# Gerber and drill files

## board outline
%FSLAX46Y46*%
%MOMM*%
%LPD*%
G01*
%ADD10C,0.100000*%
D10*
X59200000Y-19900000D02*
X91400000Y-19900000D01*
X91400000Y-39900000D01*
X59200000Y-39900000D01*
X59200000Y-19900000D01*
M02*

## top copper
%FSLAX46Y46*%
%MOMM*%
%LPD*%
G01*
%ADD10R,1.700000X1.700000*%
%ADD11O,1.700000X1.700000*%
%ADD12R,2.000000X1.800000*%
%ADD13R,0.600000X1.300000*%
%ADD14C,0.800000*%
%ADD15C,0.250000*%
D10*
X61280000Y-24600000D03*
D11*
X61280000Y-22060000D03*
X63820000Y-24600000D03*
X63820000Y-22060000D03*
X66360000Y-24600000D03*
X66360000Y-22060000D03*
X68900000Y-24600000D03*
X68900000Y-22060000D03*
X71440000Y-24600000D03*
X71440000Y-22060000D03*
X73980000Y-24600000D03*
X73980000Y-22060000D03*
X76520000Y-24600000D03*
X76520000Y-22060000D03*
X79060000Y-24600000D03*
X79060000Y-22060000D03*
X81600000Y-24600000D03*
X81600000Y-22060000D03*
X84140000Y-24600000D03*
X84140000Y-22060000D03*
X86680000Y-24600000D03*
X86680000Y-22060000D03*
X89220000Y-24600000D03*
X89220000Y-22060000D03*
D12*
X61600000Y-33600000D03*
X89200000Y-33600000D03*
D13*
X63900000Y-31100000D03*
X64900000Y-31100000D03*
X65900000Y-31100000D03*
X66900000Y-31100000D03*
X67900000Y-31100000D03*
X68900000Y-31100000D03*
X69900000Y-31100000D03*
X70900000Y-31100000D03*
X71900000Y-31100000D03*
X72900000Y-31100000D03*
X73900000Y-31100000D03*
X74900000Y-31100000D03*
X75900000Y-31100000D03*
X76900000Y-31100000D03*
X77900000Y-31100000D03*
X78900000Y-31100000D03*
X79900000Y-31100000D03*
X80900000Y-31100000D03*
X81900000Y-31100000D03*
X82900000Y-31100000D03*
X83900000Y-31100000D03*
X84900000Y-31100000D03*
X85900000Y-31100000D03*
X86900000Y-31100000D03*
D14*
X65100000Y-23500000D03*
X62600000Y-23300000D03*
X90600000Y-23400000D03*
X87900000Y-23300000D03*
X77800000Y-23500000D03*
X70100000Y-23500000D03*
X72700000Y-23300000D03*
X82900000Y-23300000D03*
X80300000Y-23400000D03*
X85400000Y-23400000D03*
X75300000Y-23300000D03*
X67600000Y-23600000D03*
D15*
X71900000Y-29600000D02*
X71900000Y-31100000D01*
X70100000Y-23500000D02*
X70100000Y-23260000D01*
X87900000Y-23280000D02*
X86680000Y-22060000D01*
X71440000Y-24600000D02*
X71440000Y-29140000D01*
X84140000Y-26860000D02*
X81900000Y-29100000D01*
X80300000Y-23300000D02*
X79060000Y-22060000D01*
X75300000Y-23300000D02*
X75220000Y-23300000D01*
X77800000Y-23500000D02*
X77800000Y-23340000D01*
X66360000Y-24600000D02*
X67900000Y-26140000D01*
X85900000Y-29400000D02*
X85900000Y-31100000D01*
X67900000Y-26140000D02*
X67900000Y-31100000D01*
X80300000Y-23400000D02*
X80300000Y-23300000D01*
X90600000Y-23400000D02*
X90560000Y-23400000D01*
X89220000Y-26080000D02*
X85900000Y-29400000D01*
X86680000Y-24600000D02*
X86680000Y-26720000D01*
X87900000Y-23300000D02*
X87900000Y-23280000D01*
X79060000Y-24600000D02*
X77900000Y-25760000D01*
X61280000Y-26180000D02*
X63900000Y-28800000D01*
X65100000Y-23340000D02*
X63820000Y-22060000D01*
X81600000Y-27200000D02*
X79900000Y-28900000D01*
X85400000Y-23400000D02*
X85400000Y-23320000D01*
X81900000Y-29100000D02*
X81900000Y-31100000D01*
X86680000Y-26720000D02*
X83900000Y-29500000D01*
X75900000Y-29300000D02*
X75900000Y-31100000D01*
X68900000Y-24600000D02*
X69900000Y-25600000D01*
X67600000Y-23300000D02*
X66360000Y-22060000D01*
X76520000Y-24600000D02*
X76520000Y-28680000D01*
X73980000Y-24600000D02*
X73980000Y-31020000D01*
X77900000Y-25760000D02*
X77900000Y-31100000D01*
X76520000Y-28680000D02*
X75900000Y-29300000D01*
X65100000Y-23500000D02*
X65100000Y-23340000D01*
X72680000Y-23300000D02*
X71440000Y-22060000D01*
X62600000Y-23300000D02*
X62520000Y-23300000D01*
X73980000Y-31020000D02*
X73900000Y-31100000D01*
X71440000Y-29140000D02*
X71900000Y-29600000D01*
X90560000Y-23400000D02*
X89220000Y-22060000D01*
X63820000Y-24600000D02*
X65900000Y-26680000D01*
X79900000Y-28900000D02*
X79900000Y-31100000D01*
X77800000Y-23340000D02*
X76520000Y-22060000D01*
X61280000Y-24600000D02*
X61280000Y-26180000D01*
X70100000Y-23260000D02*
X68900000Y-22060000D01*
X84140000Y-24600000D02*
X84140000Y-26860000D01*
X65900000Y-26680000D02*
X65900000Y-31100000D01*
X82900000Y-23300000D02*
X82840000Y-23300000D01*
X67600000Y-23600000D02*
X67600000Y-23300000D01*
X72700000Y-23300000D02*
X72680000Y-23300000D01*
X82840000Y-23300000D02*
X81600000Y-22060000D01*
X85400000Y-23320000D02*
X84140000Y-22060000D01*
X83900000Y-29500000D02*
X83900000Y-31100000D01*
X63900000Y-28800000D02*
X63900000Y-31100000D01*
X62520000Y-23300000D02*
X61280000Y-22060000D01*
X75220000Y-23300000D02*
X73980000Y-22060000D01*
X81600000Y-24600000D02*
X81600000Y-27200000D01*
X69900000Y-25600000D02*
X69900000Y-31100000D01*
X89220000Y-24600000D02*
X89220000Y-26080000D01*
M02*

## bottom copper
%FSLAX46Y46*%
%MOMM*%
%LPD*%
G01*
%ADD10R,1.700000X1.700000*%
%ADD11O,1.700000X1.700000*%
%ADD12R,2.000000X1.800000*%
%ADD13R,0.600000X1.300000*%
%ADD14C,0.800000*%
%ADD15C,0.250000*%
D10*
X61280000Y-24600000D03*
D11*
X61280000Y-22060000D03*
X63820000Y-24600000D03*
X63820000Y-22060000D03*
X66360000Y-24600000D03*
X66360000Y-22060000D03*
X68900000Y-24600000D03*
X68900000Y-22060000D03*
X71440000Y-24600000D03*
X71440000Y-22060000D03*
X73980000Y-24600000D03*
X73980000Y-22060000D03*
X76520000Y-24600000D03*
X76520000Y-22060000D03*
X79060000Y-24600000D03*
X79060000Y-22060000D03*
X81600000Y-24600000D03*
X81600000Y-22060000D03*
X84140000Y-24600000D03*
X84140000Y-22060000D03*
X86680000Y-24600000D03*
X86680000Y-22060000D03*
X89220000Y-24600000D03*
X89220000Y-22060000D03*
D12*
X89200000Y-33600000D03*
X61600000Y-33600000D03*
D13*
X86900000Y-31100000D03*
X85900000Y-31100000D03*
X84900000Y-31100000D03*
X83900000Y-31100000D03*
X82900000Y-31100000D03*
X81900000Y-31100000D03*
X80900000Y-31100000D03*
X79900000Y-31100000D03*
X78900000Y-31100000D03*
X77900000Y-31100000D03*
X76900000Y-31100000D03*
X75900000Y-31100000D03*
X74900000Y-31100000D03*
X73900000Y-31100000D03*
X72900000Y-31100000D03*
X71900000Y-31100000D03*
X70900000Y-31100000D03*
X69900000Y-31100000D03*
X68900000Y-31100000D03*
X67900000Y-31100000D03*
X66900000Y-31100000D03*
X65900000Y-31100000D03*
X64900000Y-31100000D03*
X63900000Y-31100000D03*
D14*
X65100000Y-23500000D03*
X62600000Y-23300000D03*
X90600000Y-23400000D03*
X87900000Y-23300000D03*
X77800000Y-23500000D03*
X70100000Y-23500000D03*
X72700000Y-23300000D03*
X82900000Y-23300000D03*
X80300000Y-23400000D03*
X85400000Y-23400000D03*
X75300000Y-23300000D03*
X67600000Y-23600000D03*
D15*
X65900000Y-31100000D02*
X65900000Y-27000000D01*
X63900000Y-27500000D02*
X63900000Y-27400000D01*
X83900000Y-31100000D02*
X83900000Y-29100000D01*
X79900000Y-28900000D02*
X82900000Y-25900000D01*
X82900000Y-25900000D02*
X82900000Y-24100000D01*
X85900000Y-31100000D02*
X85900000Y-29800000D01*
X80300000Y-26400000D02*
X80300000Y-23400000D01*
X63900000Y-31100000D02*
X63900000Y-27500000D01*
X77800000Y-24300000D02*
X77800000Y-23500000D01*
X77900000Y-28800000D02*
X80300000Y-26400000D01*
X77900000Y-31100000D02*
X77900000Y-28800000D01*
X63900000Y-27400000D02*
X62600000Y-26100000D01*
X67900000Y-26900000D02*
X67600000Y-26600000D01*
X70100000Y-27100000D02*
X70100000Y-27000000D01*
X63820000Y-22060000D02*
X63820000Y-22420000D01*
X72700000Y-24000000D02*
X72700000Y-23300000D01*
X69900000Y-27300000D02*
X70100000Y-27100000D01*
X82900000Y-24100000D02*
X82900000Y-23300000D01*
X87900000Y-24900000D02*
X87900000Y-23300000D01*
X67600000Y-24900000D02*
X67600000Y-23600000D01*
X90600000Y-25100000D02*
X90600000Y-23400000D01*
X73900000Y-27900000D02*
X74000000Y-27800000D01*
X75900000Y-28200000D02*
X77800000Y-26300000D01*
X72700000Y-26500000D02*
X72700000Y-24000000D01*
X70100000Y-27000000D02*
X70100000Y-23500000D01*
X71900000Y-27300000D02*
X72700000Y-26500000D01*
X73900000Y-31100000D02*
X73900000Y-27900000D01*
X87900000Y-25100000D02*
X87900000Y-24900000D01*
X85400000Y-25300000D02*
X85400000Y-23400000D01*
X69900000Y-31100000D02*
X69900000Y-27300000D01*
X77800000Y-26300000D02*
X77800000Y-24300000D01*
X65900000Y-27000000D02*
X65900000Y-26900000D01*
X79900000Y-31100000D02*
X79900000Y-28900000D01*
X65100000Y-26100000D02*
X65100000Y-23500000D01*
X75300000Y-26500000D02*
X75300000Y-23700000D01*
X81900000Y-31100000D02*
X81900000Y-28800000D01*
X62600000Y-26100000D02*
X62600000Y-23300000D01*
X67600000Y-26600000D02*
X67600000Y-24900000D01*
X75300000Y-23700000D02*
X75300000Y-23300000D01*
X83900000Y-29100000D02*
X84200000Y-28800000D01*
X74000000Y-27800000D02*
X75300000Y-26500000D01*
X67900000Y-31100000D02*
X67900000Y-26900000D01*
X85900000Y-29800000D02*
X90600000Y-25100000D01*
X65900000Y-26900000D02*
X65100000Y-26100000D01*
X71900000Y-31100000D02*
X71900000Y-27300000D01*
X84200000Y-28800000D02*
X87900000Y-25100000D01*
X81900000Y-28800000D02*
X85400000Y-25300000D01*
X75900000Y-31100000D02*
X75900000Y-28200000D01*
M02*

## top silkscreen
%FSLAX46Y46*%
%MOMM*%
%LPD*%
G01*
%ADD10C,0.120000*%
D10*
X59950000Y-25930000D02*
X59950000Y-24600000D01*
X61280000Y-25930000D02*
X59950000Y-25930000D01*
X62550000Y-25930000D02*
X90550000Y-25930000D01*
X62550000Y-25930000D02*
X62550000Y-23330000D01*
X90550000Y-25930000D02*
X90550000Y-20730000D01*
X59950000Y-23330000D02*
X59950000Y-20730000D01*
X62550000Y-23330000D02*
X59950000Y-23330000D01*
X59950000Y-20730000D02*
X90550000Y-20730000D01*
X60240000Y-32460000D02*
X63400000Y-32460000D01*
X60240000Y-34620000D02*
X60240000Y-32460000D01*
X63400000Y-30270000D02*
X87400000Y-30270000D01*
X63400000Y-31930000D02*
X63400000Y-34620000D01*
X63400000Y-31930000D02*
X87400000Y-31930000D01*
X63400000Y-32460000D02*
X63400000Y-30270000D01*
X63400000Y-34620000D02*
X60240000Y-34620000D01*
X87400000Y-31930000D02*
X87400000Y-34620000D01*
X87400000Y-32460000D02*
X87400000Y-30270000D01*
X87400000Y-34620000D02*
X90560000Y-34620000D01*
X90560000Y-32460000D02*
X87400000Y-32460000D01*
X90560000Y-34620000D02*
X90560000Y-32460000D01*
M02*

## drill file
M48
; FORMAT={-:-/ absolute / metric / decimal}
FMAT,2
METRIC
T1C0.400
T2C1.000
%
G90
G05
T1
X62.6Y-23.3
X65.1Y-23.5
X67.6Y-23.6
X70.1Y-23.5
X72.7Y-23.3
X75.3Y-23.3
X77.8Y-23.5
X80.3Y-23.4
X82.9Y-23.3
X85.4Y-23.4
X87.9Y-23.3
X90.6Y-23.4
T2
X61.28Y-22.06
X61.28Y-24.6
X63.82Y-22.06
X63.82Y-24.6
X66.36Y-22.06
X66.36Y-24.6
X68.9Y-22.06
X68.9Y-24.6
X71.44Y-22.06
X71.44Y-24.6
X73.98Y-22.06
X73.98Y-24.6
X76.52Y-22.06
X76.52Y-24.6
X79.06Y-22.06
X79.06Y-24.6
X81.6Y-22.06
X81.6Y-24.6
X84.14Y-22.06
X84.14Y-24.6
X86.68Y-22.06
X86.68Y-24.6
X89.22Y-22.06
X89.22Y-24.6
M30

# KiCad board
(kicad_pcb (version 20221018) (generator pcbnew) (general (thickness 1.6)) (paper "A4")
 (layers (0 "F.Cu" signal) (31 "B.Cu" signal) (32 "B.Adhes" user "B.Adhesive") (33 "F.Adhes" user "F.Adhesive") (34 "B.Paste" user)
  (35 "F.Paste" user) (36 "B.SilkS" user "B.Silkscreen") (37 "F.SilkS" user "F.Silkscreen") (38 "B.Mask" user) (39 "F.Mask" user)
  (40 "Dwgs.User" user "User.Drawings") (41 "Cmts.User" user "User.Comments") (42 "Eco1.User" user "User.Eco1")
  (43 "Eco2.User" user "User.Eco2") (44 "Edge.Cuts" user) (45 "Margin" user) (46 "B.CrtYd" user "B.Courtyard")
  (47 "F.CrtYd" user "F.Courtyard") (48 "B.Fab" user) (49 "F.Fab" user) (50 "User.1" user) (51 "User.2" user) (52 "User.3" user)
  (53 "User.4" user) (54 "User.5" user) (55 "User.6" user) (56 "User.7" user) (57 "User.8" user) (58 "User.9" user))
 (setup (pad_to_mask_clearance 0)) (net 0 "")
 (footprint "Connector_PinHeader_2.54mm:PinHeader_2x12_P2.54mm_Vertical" (layer "F.Cu") (at 61.28 24.6 90)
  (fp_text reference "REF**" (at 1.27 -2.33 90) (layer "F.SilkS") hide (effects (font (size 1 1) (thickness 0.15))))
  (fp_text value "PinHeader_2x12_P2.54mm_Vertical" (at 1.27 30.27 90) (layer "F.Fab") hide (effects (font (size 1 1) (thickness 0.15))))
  (fp_line (start -1.33 -1.33) (end 0 -1.33) (stroke (width 0.12) (type solid)) (layer "F.SilkS"))
  (fp_line (start -1.33 0) (end -1.33 -1.33) (stroke (width 0.12) (type solid)) (layer "F.SilkS"))
  (fp_line (start -1.33 1.27) (end -1.33 29.27) (stroke (width 0.12) (type solid)) (layer "F.SilkS"))
  (fp_line (start -1.33 1.27) (end 1.27 1.27) (stroke (width 0.12) (type solid)) (layer "F.SilkS"))
  (fp_line (start -1.33 29.27) (end 3.87 29.27) (stroke (width 0.12) (type solid)) (layer "F.SilkS"))
  (fp_line (start 1.27 -1.33) (end 3.87 -1.33) (stroke (width 0.12) (type solid)) (layer "F.SilkS"))
  (fp_line (start 1.27 1.27) (end 1.27 -1.33) (stroke (width 0.12) (type solid)) (layer "F.SilkS"))
  (fp_line (start 3.87 -1.33) (end 3.87 29.27) (stroke (width 0.12) (type solid)) (layer "F.SilkS"))
  (pad "1" thru_hole rect (at 0 0 90) (size 1.7 1.7) (drill 1) (layers "*.Cu" "*.Mask"))
  (pad "2" thru_hole oval (at 2.54 0 90) (size 1.7 1.7) (drill 1) (layers "*.Cu" "*.Mask"))
  (pad "3" thru_hole oval (at 0 2.54 90) (size 1.7 1.7) (drill 1) (layers "*.Cu" "*.Mask"))
  (pad "4" thru_hole oval (at 2.54 2.54 90) (size 1.7 1.7) (drill 1) (layers "*.Cu" "*.Mask"))
  (pad "5" thru_hole oval (at 0 5.08 90) (size 1.7 1.7) (drill 1) (layers "*.Cu" "*.Mask"))
  (pad "6" thru_hole oval (at 2.54 5.08 90) (size 1.7 1.7) (drill 1) (layers "*.Cu" "*.Mask"))
  (pad "7" thru_hole oval (at 0 7.62 90) (size 1.7 1.7) (drill 1) (layers "*.Cu" "*.Mask"))
  (pad "8" thru_hole oval (at 2.54 7.62 90) (size 1.7 1.7) (drill 1) (layers "*.Cu" "*.Mask"))
  (pad "9" thru_hole oval (at 0 10.16 90) (size 1.7 1.7) (drill 1) (layers "*.Cu" "*.Mask"))
  (pad "10" thru_hole oval (at 2.54 10.16 90) (size 1.7 1.7) (drill 1) (layers "*.Cu" "*.Mask"))
  (pad "11" thru_hole oval (at 0 12.7 90) (size 1.7 1.7) (drill 1) (layers "*.Cu" "*.Mask"))
  (pad "12" thru_hole oval (at 2.54 12.7 90) (size 1.7 1.7) (drill 1) (layers "*.Cu" "*.Mask"))
  (pad "13" thru_hole oval (at 0 15.24 90) (size 1.7 1.7) (drill 1) (layers "*.Cu" "*.Mask"))
  (pad "14" thru_hole oval (at 2.54 15.24 90) (size 1.7 1.7) (drill 1) (layers "*.Cu" "*.Mask"))
  (pad "15" thru_hole oval (at 0 17.78 90) (size 1.7 1.7) (drill 1) (layers "*.Cu" "*.Mask"))
  (pad "16" thru_hole oval (at 2.54 17.78 90) (size 1.7 1.7) (drill 1) (layers "*.Cu" "*.Mask"))
  (pad "17" thru_hole oval (at 0 20.32 90) (size 1.7 1.7) (drill 1) (layers "*.Cu" "*.Mask"))
  (pad "18" thru_hole oval (at 2.54 20.32 90) (size 1.7 1.7) (drill 1) (layers "*.Cu" "*.Mask"))
  (pad "19" thru_hole oval (at 0 22.86 90) (size 1.7 1.7) (drill 1) (layers "*.Cu" "*.Mask"))
  (pad "20" thru_hole oval (at 2.54 22.86 90) (size 1.7 1.7) (drill 1) (layers "*.Cu" "*.Mask"))
  (pad "21" thru_hole oval (at 0 25.4 90) (size 1.7 1.7) (drill 1) (layers "*.Cu" "*.Mask"))
  (pad "22" thru_hole oval (at 2.54 25.4 90) (size 1.7 1.7) (drill 1) (layers "*.Cu" "*.Mask"))
  (pad "23" thru_hole oval (at 0 27.94 90) (size 1.7 1.7) (drill 1) (layers "*.Cu" "*.Mask"))
  (pad "24" thru_hole oval (at 2.54 27.94 90) (size 1.7 1.7) (drill 1) (layers "*.Cu" "*.Mask")))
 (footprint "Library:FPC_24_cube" (layer "F.Cu") (at 75.4 31.1)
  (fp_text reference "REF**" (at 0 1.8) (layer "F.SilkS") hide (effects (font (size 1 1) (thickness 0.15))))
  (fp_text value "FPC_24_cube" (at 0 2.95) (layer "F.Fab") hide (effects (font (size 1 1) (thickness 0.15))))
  (fp_line (start -15.16 1.36) (end -12 1.36) (stroke (width 0.12) (type default)) (layer "F.SilkS"))
  (fp_line (start -15.16 3.52) (end -15.16 1.36) (stroke (width 0.12) (type default)) (layer "F.SilkS"))
  (fp_line (start -12 -0.83) (end 12 -0.83) (stroke (width 0.12) (type default)) (layer "F.SilkS"))
  (fp_line (start -12 0.83) (end -12 3.52) (stroke (width 0.12) (type default)) (layer "F.SilkS"))
  (fp_line (start -12 0.83) (end 12 0.83) (stroke (width 0.12) (type default)) (layer "F.SilkS"))
  (fp_line (start -12 1.36) (end -12 -0.83) (stroke (width 0.12) (type default)) (layer "F.SilkS"))
  (fp_line (start -12 3.52) (end -15.16 3.52) (stroke (width 0.12) (type default)) (layer "F.SilkS"))
  (fp_line (start 12 0.83) (end 12 3.52) (stroke (width 0.12) (type default)) (layer "F.SilkS"))
  (fp_line (start 12 1.36) (end 12 -0.83) (stroke (width 0.12) (type default)) (layer "F.SilkS"))
  (fp_line (start 12 3.52) (end 15.16 3.52) (stroke (width 0.12) (type default)) (layer "F.SilkS"))
  (fp_line (start 15.16 1.36) (end 12 1.36) (stroke (width 0.12) (type default)) (layer "F.SilkS"))
  (fp_line (start 15.16 3.52) (end 15.16 1.36) (stroke (width 0.12) (type default)) (layer "F.SilkS"))
  (pad "0" smd rect (at -13.8 2.5) (size 2 1.8) (layers "F.Cu" "F.Paste" "F.Mask") (thermal_bridge_angle 45))
  (pad "0" smd rect (at 13.8 2.5) (size 2 1.8) (layers "F.Cu" "F.Paste" "F.Mask") (thermal_bridge_angle 45))
  (pad "1" smd rect (at -11.5 0) (size 0.6 1.3) (layers "F.Cu" "F.Paste" "F.Mask") (thermal_bridge_angle 45))
  (pad "2" smd rect (at -10.5 0) (size 0.6 1.3) (layers "F.Cu" "F.Paste" "F.Mask") (thermal_bridge_angle 45))
  (pad "3" smd rect (at -9.5 0) (size 0.6 1.3) (layers "F.Cu" "F.Paste" "F.Mask") (thermal_bridge_angle 45))
  (pad "4" smd rect (at -8.5 0) (size 0.6 1.3) (layers "F.Cu" "F.Paste" "F.Mask") (thermal_bridge_angle 45))
  (pad "5" smd rect (at -7.5 0) (size 0.6 1.3) (layers "F.Cu" "F.Paste" "F.Mask") (thermal_bridge_angle 45))
  (pad "6" smd rect (at -6.5 0) (size 0.6 1.3) (layers "F.Cu" "F.Paste" "F.Mask") (thermal_bridge_angle 45))
  (pad "7" smd rect (at -5.5 0) (size 0.6 1.3) (layers "F.Cu" "F.Paste" "F.Mask") (thermal_bridge_angle 45))
  (pad "8" smd rect (at -4.5 0) (size 0.6 1.3) (layers "F.Cu" "F.Paste" "F.Mask") (thermal_bridge_angle 45))
  (pad "9" smd rect (at -3.5 0) (size 0.6 1.3) (layers "F.Cu" "F.Paste" "F.Mask") (thermal_bridge_angle 45))
  (pad "10" smd rect (at -2.5 0) (size 0.6 1.3) (layers "F.Cu" "F.Paste" "F.Mask") (thermal_bridge_angle 45))
  (pad "11" smd rect (at -1.5 0) (size 0.6 1.3) (layers "F.Cu" "F.Paste" "F.Mask") (thermal_bridge_angle 45))
  (pad "12" smd rect (at -0.5 0) (size 0.6 1.3) (layers "F.Cu" "F.Paste" "F.Mask") (thermal_bridge_angle 45))
  (pad "13" smd rect (at 0.5 0) (size 0.6 1.3) (layers "F.Cu" "F.Paste" "F.Mask") (thermal_bridge_angle 45))
  (pad "14" smd rect (at 1.5 0) (size 0.6 1.3) (layers "F.Cu" "F.Paste" "F.Mask") (thermal_bridge_angle 45))
  (pad "15" smd rect (at 2.5 0) (size 0.6 1.3) (layers "F.Cu" "F.Paste" "F.Mask") (thermal_bridge_angle 45))
  (pad "16" smd rect (at 3.5 0) (size 0.6 1.3) (layers "F.Cu" "F.Paste" "F.Mask") (thermal_bridge_angle 45))
  (pad "17" smd rect (at 4.5 0) (size 0.6 1.3) (layers "F.Cu" "F.Paste" "F.Mask") (thermal_bridge_angle 45))
  (pad "18" smd rect (at 5.5 0) (size 0.6 1.3) (layers "F.Cu" "F.Paste" "F.Mask") (thermal_bridge_angle 45))
  (pad "19" smd rect (at 6.5 0) (size 0.6 1.3) (layers "F.Cu" "F.Paste" "F.Mask") (thermal_bridge_angle 45))
  (pad "20" smd rect (at 7.5 0) (size 0.6 1.3) (layers "F.Cu" "F.Paste" "F.Mask") (thermal_bridge_angle 45))
  (pad "21" smd rect (at 8.5 0) (size 0.6 1.3) (layers "F.Cu" "F.Paste" "F.Mask") (thermal_bridge_angle 45))
  (pad "22" smd rect (at 9.5 0) (size 0.6 1.3) (layers "F.Cu" "F.Paste" "F.Mask") (thermal_bridge_angle 45))
  (pad "23" smd rect (at 10.5 0) (size 0.6 1.3) (layers "F.Cu" "F.Paste" "F.Mask") (thermal_bridge_angle 45))
  (pad "24" smd rect (at 11.5 0) (size 0.6 1.3) (layers "F.Cu" "F.Paste" "F.Mask") (thermal_bridge_angle 45)))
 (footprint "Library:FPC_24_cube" (layer "B.Cu") (at 75.4 31.1 180)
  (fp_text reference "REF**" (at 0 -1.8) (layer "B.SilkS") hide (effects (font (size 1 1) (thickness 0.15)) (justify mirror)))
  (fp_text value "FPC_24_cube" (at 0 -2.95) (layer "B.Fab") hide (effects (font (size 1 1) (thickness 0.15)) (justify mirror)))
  (pad "0" smd rect (at -13.8 -2.5 180) (size 2 1.8) (layers "B.Cu" "B.Paste" "B.Mask") (thermal_bridge_angle 45))
  (pad "0" smd rect (at 13.8 -2.5 180) (size 2 1.8) (layers "B.Cu" "B.Paste" "B.Mask") (thermal_bridge_angle 45))
  (pad "1" smd rect (at -11.5 0 180) (size 0.6 1.3) (layers "B.Cu" "B.Paste" "B.Mask") (thermal_bridge_angle 45))
  (pad "2" smd rect (at -10.5 0 180) (size 0.6 1.3) (layers "B.Cu" "B.Paste" "B.Mask") (thermal_bridge_angle 45))
  (pad "3" smd rect (at -9.5 0 180) (size 0.6 1.3) (layers "B.Cu" "B.Paste" "B.Mask") (thermal_bridge_angle 45))
  (pad "4" smd rect (at -8.5 0 180) (size 0.6 1.3) (layers "B.Cu" "B.Paste" "B.Mask") (thermal_bridge_angle 45))
  (pad "5" smd rect (at -7.5 0 180) (size 0.6 1.3) (layers "B.Cu" "B.Paste" "B.Mask") (thermal_bridge_angle 45))
  (pad "6" smd rect (at -6.5 0 180) (size 0.6 1.3) (layers "B.Cu" "B.Paste" "B.Mask") (thermal_bridge_angle 45))
  (pad "7" smd rect (at -5.5 0 180) (size 0.6 1.3) (layers "B.Cu" "B.Paste" "B.Mask") (thermal_bridge_angle 45))
  (pad "8" smd rect (at -4.5 0 180) (size 0.6 1.3) (layers "B.Cu" "B.Paste" "B.Mask") (thermal_bridge_angle 45))
  (pad "9" smd rect (at -3.5 0 180) (size 0.6 1.3) (layers "B.Cu" "B.Paste" "B.Mask") (thermal_bridge_angle 45))
  (pad "10" smd rect (at -2.5 0 180) (size 0.6 1.3) (layers "B.Cu" "B.Paste" "B.Mask") (thermal_bridge_angle 45))
  (pad "11" smd rect (at -1.5 0 180) (size 0.6 1.3) (layers "B.Cu" "B.Paste" "B.Mask") (thermal_bridge_angle 45))
  (pad "12" smd rect (at -0.5 0 180) (size 0.6 1.3) (layers "B.Cu" "B.Paste" "B.Mask") (thermal_bridge_angle 45))
  (pad "13" smd rect (at 0.5 0 180) (size 0.6 1.3) (layers "B.Cu" "B.Paste" "B.Mask") (thermal_bridge_angle 45))
  (pad "14" smd rect (at 1.5 0 180) (size 0.6 1.3) (layers "B.Cu" "B.Paste" "B.Mask") (thermal_bridge_angle 45))
  (pad "15" smd rect (at 2.5 0 180) (size 0.6 1.3) (layers "B.Cu" "B.Paste" "B.Mask") (thermal_bridge_angle 45))
  (pad "16" smd rect (at 3.5 0 180) (size 0.6 1.3) (layers "B.Cu" "B.Paste" "B.Mask") (thermal_bridge_angle 45))
  (pad "17" smd rect (at 4.5 0 180) (size 0.6 1.3) (layers "B.Cu" "B.Paste" "B.Mask") (thermal_bridge_angle 45))
  (pad "18" smd rect (at 5.5 0 180) (size 0.6 1.3) (layers "B.Cu" "B.Paste" "B.Mask") (thermal_bridge_angle 45))
  (pad "19" smd rect (at 6.5 0 180) (size 0.6 1.3) (layers "B.Cu" "B.Paste" "B.Mask") (thermal_bridge_angle 45))
  (pad "20" smd rect (at 7.5 0 180) (size 0.6 1.3) (layers "B.Cu" "B.Paste" "B.Mask") (thermal_bridge_angle 45))
  (pad "21" smd rect (at 8.5 0 180) (size 0.6 1.3) (layers "B.Cu" "B.Paste" "B.Mask") (thermal_bridge_angle 45))
  (pad "22" smd rect (at 9.5 0 180) (size 0.6 1.3) (layers "B.Cu" "B.Paste" "B.Mask") (thermal_bridge_angle 45))
  (pad "23" smd rect (at 10.5 0 180) (size 0.6 1.3) (layers "B.Cu" "B.Paste" "B.Mask") (thermal_bridge_angle 45))
  (pad "24" smd rect (at 11.5 0 180) (size 0.6 1.3) (layers "B.Cu" "B.Paste" "B.Mask") (thermal_bridge_angle 45)))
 (gr_rect (start 59.2 19.9) (end 91.4 39.9) (stroke (width 0.1) (type default)) (fill none) (layer "Edge.Cuts"))
 (segment (start 71.9 29.6) (end 71.9 31.1) (width 0.25) (layer "F.Cu") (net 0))
 (segment (start 70.1 23.5) (end 70.1 23.26) (width 0.25) (layer "F.Cu") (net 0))
 (segment (start 87.9 23.28) (end 86.68 22.06) (width 0.25) (layer "F.Cu") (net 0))
 (segment (start 71.44 24.6) (end 71.44 29.14) (width 0.25) (layer "F.Cu") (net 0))
 (segment (start 84.14 26.86) (end 81.9 29.1) (width 0.25) (layer "F.Cu") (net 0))
 (segment (start 80.3 23.3) (end 79.06 22.06) (width 0.25) (layer "F.Cu") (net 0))
 (segment (start 75.3 23.3) (end 75.22 23.3) (width 0.25) (layer "F.Cu") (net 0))
 (segment (start 77.8 23.5) (end 77.8 23.34) (width 0.25) (layer "F.Cu") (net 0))
 (segment (start 66.36 24.6) (end 67.9 26.14) (width 0.25) (layer "F.Cu") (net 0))
 (segment (start 85.9 29.4) (end 85.9 31.1) (width 0.25) (layer "F.Cu") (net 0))
 (segment (start 67.9 26.14) (end 67.9 31.1) (width 0.25) (layer "F.Cu") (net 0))
 (segment (start 80.3 23.4) (end 80.3 23.3) (width 0.25) (layer "F.Cu") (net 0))
 (segment (start 90.6 23.4) (end 90.56 23.4) (width 0.25) (layer "F.Cu") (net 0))
 (segment (start 89.22 26.08) (end 85.9 29.4) (width 0.25) (layer "F.Cu") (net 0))
 (segment (start 86.68 24.6) (end 86.68 26.72) (width 0.25) (layer "F.Cu") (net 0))
 (segment (start 87.9 23.3) (end 87.9 23.28) (width 0.25) (layer "F.Cu") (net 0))
 (segment (start 79.06 24.6) (end 77.9 25.76) (width 0.25) (layer "F.Cu") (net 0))
 (segment (start 61.28 26.18) (end 63.9 28.8) (width 0.25) (layer "F.Cu") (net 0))
 (segment (start 65.1 23.34) (end 63.82 22.06) (width 0.25) (layer "F.Cu") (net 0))
 (segment (start 81.6 27.2) (end 79.9 28.9) (width 0.25) (layer "F.Cu") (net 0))
 (segment (start 85.4 23.4) (end 85.4 23.32) (width 0.25) (layer "F.Cu") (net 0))
 (segment (start 81.9 29.1) (end 81.9 31.1) (width 0.25) (layer "F.Cu") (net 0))
 (segment (start 86.68 26.72) (end 83.9 29.5) (width 0.25) (layer "F.Cu") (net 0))
 (segment (start 75.9 29.3) (end 75.9 31.1) (width 0.25) (layer "F.Cu") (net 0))
 (segment (start 68.9 24.6) (end 69.9 25.6) (width 0.25) (layer "F.Cu") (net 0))
 (segment (start 67.6 23.3) (end 66.36 22.06) (width 0.25) (layer "F.Cu") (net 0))
 (segment (start 76.52 24.6) (end 76.52 28.68) (width 0.25) (layer "F.Cu") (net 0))
 (segment (start 73.98 24.6) (end 73.98 31.02) (width 0.25) (layer "F.Cu") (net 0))
 (segment (start 77.9 25.76) (end 77.9 31.1) (width 0.25) (layer "F.Cu") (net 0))
 (segment (start 76.52 28.68) (end 75.9 29.3) (width 0.25) (layer "F.Cu") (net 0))
 (segment (start 65.1 23.5) (end 65.1 23.34) (width 0.25) (layer "F.Cu") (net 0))
 (segment (start 72.68 23.3) (end 71.44 22.06) (width 0.25) (layer "F.Cu") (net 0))
 (segment (start 62.6 23.3) (end 62.52 23.3) (width 0.25) (layer "F.Cu") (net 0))
 (segment (start 73.98 31.02) (end 73.9 31.1) (width 0.25) (layer "F.Cu") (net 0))
 (segment (start 71.44 29.14) (end 71.9 29.6) (width 0.25) (layer "F.Cu") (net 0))
 (segment (start 90.56 23.4) (end 89.22 22.06) (width 0.25) (layer "F.Cu") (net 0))
 (segment (start 63.82 24.6) (end 65.9 26.68) (width 0.25) (layer "F.Cu") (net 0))
 (segment (start 79.9 28.9) (end 79.9 31.1) (width 0.25) (layer "F.Cu") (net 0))
 (segment (start 77.8 23.34) (end 76.52 22.06) (width 0.25) (layer "F.Cu") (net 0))
 (segment (start 61.28 24.6) (end 61.28 26.18) (width 0.25) (layer "F.Cu") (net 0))
 (segment (start 70.1 23.26) (end 68.9 22.06) (width 0.25) (layer "F.Cu") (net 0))
 (segment (start 84.14 24.6) (end 84.14 26.86) (width 0.25) (layer "F.Cu") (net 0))
 (segment (start 65.9 26.68) (end 65.9 31.1) (width 0.25) (layer "F.Cu") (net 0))
 (segment (start 82.9 23.3) (end 82.84 23.3) (width 0.25) (layer "F.Cu") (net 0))
 (segment (start 67.6 23.6) (end 67.6 23.3) (width 0.25) (layer "F.Cu") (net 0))
 (segment (start 72.7 23.3) (end 72.68 23.3) (width 0.25) (layer "F.Cu") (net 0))
 (segment (start 82.84 23.3) (end 81.6 22.06) (width 0.25) (layer "F.Cu") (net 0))
 (segment (start 85.4 23.32) (end 84.14 22.06) (width 0.25) (layer "F.Cu") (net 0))
 (segment (start 83.9 29.5) (end 83.9 31.1) (width 0.25) (layer "F.Cu") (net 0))
 (segment (start 63.9 28.8) (end 63.9 31.1) (width 0.25) (layer "F.Cu") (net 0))
 (segment (start 62.52 23.3) (end 61.28 22.06) (width 0.25) (layer "F.Cu") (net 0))
 (segment (start 75.22 23.3) (end 73.98 22.06) (width 0.25) (layer "F.Cu") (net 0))
 (segment (start 81.6 24.6) (end 81.6 27.2) (width 0.25) (layer "F.Cu") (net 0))
 (segment (start 69.9 25.6) (end 69.9 31.1) (width 0.25) (layer "F.Cu") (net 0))
 (segment (start 89.22 24.6) (end 89.22 26.08) (width 0.25) (layer "F.Cu") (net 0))
 (via (at 65.1 23.5) (size 0.8) (drill 0.4) (layers "F.Cu" "B.Cu") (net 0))
 (via (at 62.6 23.3) (size 0.8) (drill 0.4) (layers "F.Cu" "B.Cu") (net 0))
 (via (at 90.6 23.4) (size 0.8) (drill 0.4) (layers "F.Cu" "B.Cu") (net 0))
 (via (at 87.9 23.3) (size 0.8) (drill 0.4) (layers "F.Cu" "B.Cu") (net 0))
 (via (at 77.8 23.5) (size 0.8) (drill 0.4) (layers "F.Cu" "B.Cu") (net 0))
 (via (at 70.1 23.5) (size 0.8) (drill 0.4) (layers "F.Cu" "B.Cu") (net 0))
 (via (at 72.7 23.3) (size 0.8) (drill 0.4) (layers "F.Cu" "B.Cu") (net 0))
 (via (at 82.9 23.3) (size 0.8) (drill 0.4) (layers "F.Cu" "B.Cu") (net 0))
 (via (at 80.3 23.4) (size 0.8) (drill 0.4) (layers "F.Cu" "B.Cu") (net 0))
 (via (at 85.4 23.4) (size 0.8) (drill 0.4) (layers "F.Cu" "B.Cu") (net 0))
 (via (at 75.3 23.3) (size 0.8) (drill 0.4) (layers "F.Cu" "B.Cu") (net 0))
 (via (at 67.6 23.6) (size 0.8) (drill 0.4) (layers "F.Cu" "B.Cu") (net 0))
 (segment (start 65.9 31.1) (end 65.9 27) (width 0.25) (layer "B.Cu") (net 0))
 (segment (start 63.9 27.5) (end 63.9 27.4) (width 0.25) (layer "B.Cu") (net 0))
 (segment (start 83.9 31.1) (end 83.9 29.1) (width 0.25) (layer "B.Cu") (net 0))
 (segment (start 79.9 28.9) (end 82.9 25.9) (width 0.25) (layer "B.Cu") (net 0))
 (segment (start 82.9 25.9) (end 82.9 24.1) (width 0.25) (layer "B.Cu") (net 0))
 (segment (start 85.9 31.1) (end 85.9 29.8) (width 0.25) (layer "B.Cu") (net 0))
 (segment (start 80.3 26.4) (end 80.3 23.4) (width 0.25) (layer "B.Cu") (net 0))
 (segment (start 63.9 31.1) (end 63.9 27.5) (width 0.25) (layer "B.Cu") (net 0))
 (segment (start 77.8 24.3) (end 77.8 23.5) (width 0.25) (layer "B.Cu") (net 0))
 (segment (start 77.9 28.8) (end 80.3 26.4) (width 0.25) (layer "B.Cu") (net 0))
 (segment (start 77.9 31.1) (end 77.9 28.8) (width 0.25) (layer "B.Cu") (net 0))
 (segment (start 63.9 27.4) (end 62.6 26.1) (width 0.25) (layer "B.Cu") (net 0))
 (segment (start 67.9 26.9) (end 67.6 26.6) (width 0.25) (layer "B.Cu") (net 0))
 (segment (start 70.1 27.1) (end 70.1 27) (width 0.25) (layer "B.Cu") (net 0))
 (segment (start 63.82 22.06) (end 63.82 22.42) (width 0.25) (layer "B.Cu") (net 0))
 (segment (start 72.7 24) (end 72.7 23.3) (width 0.25) (layer "B.Cu") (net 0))
 (segment (start 69.9 27.3) (end 70.1 27.1) (width 0.25) (layer "B.Cu") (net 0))
 (segment (start 82.9 24.1) (end 82.9 23.3) (width 0.25) (layer "B.Cu") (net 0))
 (segment (start 87.9 24.9) (end 87.9 23.3) (width 0.25) (layer "B.Cu") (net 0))
 (segment (start 67.6 24.9) (end 67.6 23.6) (width 0.25) (layer "B.Cu") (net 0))
 (segment (start 90.6 25.1) (end 90.6 23.4) (width 0.25) (layer "B.Cu") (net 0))
 (segment (start 73.9 27.9) (end 74 27.8) (width 0.25) (layer "B.Cu") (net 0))
 (segment (start 75.9 28.2) (end 77.8 26.3) (width 0.25) (layer "B.Cu") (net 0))
 (segment (start 72.7 26.5) (end 72.7 24) (width 0.25) (layer "B.Cu") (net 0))
 (segment (start 70.1 27) (end 70.1 23.5) (width 0.25) (layer "B.Cu") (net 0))
 (segment (start 71.9 27.3) (end 72.7 26.5) (width 0.25) (layer "B.Cu") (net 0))
 (segment (start 73.9 31.1) (end 73.9 27.9) (width 0.25) (layer "B.Cu") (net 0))
 (segment (start 87.9 25.1) (end 87.9 24.9) (width 0.25) (layer "B.Cu") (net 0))
 (segment (start 85.4 25.3) (end 85.4 23.4) (width 0.25) (layer "B.Cu") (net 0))
 (segment (start 69.9 31.1) (end 69.9 27.3) (width 0.25) (layer "B.Cu") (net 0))
 (segment (start 77.8 26.3) (end 77.8 24.3) (width 0.25) (layer "B.Cu") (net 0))
 (segment (start 65.9 27) (end 65.9 26.9) (width 0.25) (layer "B.Cu") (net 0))
 (segment (start 79.9 31.1) (end 79.9 28.9) (width 0.25) (layer "B.Cu") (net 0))
 (segment (start 65.1 26.1) (end 65.1 23.5) (width 0.25) (layer "B.Cu") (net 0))
 (segment (start 75.3 26.5) (end 75.3 23.7) (width 0.25) (layer "B.Cu") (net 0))
 (segment (start 81.9 31.1) (end 81.9 28.8) (width 0.25) (layer "B.Cu") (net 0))
 (segment (start 62.6 26.1) (end 62.6 23.3) (width 0.25) (layer "B.Cu") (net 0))
 (segment (start 67.6 26.6) (end 67.6 24.9) (width 0.25) (layer "B.Cu") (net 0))
 (segment (start 75.3 23.7) (end 75.3 23.3) (width 0.25) (layer "B.Cu") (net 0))
 (segment (start 83.9 29.1) (end 84.2 28.8) (width 0.25) (layer "B.Cu") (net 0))
 (segment (start 74 27.8) (end 75.3 26.5) (width 0.25) (layer "B.Cu") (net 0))
 (segment (start 67.9 31.1) (end 67.9 26.9) (width 0.25) (layer "B.Cu") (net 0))
 (segment (start 85.9 29.8) (end 90.6 25.1) (width 0.25) (layer "B.Cu") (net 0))
 (segment (start 65.9 26.9) (end 65.1 26.1) (width 0.25) (layer "B.Cu") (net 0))
 (segment (start 71.9 31.1) (end 71.9 27.3) (width 0.25) (layer "B.Cu") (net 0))
 (segment (start 84.2 28.8) (end 87.9 25.1) (width 0.25) (layer "B.Cu") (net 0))
 (segment (start 81.9 28.8) (end 85.4 25.3) (width 0.25) (layer "B.Cu") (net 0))
 (segment (start 75.9 31.1) (end 75.9 28.2) (width 0.25) (layer "B.Cu") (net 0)))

